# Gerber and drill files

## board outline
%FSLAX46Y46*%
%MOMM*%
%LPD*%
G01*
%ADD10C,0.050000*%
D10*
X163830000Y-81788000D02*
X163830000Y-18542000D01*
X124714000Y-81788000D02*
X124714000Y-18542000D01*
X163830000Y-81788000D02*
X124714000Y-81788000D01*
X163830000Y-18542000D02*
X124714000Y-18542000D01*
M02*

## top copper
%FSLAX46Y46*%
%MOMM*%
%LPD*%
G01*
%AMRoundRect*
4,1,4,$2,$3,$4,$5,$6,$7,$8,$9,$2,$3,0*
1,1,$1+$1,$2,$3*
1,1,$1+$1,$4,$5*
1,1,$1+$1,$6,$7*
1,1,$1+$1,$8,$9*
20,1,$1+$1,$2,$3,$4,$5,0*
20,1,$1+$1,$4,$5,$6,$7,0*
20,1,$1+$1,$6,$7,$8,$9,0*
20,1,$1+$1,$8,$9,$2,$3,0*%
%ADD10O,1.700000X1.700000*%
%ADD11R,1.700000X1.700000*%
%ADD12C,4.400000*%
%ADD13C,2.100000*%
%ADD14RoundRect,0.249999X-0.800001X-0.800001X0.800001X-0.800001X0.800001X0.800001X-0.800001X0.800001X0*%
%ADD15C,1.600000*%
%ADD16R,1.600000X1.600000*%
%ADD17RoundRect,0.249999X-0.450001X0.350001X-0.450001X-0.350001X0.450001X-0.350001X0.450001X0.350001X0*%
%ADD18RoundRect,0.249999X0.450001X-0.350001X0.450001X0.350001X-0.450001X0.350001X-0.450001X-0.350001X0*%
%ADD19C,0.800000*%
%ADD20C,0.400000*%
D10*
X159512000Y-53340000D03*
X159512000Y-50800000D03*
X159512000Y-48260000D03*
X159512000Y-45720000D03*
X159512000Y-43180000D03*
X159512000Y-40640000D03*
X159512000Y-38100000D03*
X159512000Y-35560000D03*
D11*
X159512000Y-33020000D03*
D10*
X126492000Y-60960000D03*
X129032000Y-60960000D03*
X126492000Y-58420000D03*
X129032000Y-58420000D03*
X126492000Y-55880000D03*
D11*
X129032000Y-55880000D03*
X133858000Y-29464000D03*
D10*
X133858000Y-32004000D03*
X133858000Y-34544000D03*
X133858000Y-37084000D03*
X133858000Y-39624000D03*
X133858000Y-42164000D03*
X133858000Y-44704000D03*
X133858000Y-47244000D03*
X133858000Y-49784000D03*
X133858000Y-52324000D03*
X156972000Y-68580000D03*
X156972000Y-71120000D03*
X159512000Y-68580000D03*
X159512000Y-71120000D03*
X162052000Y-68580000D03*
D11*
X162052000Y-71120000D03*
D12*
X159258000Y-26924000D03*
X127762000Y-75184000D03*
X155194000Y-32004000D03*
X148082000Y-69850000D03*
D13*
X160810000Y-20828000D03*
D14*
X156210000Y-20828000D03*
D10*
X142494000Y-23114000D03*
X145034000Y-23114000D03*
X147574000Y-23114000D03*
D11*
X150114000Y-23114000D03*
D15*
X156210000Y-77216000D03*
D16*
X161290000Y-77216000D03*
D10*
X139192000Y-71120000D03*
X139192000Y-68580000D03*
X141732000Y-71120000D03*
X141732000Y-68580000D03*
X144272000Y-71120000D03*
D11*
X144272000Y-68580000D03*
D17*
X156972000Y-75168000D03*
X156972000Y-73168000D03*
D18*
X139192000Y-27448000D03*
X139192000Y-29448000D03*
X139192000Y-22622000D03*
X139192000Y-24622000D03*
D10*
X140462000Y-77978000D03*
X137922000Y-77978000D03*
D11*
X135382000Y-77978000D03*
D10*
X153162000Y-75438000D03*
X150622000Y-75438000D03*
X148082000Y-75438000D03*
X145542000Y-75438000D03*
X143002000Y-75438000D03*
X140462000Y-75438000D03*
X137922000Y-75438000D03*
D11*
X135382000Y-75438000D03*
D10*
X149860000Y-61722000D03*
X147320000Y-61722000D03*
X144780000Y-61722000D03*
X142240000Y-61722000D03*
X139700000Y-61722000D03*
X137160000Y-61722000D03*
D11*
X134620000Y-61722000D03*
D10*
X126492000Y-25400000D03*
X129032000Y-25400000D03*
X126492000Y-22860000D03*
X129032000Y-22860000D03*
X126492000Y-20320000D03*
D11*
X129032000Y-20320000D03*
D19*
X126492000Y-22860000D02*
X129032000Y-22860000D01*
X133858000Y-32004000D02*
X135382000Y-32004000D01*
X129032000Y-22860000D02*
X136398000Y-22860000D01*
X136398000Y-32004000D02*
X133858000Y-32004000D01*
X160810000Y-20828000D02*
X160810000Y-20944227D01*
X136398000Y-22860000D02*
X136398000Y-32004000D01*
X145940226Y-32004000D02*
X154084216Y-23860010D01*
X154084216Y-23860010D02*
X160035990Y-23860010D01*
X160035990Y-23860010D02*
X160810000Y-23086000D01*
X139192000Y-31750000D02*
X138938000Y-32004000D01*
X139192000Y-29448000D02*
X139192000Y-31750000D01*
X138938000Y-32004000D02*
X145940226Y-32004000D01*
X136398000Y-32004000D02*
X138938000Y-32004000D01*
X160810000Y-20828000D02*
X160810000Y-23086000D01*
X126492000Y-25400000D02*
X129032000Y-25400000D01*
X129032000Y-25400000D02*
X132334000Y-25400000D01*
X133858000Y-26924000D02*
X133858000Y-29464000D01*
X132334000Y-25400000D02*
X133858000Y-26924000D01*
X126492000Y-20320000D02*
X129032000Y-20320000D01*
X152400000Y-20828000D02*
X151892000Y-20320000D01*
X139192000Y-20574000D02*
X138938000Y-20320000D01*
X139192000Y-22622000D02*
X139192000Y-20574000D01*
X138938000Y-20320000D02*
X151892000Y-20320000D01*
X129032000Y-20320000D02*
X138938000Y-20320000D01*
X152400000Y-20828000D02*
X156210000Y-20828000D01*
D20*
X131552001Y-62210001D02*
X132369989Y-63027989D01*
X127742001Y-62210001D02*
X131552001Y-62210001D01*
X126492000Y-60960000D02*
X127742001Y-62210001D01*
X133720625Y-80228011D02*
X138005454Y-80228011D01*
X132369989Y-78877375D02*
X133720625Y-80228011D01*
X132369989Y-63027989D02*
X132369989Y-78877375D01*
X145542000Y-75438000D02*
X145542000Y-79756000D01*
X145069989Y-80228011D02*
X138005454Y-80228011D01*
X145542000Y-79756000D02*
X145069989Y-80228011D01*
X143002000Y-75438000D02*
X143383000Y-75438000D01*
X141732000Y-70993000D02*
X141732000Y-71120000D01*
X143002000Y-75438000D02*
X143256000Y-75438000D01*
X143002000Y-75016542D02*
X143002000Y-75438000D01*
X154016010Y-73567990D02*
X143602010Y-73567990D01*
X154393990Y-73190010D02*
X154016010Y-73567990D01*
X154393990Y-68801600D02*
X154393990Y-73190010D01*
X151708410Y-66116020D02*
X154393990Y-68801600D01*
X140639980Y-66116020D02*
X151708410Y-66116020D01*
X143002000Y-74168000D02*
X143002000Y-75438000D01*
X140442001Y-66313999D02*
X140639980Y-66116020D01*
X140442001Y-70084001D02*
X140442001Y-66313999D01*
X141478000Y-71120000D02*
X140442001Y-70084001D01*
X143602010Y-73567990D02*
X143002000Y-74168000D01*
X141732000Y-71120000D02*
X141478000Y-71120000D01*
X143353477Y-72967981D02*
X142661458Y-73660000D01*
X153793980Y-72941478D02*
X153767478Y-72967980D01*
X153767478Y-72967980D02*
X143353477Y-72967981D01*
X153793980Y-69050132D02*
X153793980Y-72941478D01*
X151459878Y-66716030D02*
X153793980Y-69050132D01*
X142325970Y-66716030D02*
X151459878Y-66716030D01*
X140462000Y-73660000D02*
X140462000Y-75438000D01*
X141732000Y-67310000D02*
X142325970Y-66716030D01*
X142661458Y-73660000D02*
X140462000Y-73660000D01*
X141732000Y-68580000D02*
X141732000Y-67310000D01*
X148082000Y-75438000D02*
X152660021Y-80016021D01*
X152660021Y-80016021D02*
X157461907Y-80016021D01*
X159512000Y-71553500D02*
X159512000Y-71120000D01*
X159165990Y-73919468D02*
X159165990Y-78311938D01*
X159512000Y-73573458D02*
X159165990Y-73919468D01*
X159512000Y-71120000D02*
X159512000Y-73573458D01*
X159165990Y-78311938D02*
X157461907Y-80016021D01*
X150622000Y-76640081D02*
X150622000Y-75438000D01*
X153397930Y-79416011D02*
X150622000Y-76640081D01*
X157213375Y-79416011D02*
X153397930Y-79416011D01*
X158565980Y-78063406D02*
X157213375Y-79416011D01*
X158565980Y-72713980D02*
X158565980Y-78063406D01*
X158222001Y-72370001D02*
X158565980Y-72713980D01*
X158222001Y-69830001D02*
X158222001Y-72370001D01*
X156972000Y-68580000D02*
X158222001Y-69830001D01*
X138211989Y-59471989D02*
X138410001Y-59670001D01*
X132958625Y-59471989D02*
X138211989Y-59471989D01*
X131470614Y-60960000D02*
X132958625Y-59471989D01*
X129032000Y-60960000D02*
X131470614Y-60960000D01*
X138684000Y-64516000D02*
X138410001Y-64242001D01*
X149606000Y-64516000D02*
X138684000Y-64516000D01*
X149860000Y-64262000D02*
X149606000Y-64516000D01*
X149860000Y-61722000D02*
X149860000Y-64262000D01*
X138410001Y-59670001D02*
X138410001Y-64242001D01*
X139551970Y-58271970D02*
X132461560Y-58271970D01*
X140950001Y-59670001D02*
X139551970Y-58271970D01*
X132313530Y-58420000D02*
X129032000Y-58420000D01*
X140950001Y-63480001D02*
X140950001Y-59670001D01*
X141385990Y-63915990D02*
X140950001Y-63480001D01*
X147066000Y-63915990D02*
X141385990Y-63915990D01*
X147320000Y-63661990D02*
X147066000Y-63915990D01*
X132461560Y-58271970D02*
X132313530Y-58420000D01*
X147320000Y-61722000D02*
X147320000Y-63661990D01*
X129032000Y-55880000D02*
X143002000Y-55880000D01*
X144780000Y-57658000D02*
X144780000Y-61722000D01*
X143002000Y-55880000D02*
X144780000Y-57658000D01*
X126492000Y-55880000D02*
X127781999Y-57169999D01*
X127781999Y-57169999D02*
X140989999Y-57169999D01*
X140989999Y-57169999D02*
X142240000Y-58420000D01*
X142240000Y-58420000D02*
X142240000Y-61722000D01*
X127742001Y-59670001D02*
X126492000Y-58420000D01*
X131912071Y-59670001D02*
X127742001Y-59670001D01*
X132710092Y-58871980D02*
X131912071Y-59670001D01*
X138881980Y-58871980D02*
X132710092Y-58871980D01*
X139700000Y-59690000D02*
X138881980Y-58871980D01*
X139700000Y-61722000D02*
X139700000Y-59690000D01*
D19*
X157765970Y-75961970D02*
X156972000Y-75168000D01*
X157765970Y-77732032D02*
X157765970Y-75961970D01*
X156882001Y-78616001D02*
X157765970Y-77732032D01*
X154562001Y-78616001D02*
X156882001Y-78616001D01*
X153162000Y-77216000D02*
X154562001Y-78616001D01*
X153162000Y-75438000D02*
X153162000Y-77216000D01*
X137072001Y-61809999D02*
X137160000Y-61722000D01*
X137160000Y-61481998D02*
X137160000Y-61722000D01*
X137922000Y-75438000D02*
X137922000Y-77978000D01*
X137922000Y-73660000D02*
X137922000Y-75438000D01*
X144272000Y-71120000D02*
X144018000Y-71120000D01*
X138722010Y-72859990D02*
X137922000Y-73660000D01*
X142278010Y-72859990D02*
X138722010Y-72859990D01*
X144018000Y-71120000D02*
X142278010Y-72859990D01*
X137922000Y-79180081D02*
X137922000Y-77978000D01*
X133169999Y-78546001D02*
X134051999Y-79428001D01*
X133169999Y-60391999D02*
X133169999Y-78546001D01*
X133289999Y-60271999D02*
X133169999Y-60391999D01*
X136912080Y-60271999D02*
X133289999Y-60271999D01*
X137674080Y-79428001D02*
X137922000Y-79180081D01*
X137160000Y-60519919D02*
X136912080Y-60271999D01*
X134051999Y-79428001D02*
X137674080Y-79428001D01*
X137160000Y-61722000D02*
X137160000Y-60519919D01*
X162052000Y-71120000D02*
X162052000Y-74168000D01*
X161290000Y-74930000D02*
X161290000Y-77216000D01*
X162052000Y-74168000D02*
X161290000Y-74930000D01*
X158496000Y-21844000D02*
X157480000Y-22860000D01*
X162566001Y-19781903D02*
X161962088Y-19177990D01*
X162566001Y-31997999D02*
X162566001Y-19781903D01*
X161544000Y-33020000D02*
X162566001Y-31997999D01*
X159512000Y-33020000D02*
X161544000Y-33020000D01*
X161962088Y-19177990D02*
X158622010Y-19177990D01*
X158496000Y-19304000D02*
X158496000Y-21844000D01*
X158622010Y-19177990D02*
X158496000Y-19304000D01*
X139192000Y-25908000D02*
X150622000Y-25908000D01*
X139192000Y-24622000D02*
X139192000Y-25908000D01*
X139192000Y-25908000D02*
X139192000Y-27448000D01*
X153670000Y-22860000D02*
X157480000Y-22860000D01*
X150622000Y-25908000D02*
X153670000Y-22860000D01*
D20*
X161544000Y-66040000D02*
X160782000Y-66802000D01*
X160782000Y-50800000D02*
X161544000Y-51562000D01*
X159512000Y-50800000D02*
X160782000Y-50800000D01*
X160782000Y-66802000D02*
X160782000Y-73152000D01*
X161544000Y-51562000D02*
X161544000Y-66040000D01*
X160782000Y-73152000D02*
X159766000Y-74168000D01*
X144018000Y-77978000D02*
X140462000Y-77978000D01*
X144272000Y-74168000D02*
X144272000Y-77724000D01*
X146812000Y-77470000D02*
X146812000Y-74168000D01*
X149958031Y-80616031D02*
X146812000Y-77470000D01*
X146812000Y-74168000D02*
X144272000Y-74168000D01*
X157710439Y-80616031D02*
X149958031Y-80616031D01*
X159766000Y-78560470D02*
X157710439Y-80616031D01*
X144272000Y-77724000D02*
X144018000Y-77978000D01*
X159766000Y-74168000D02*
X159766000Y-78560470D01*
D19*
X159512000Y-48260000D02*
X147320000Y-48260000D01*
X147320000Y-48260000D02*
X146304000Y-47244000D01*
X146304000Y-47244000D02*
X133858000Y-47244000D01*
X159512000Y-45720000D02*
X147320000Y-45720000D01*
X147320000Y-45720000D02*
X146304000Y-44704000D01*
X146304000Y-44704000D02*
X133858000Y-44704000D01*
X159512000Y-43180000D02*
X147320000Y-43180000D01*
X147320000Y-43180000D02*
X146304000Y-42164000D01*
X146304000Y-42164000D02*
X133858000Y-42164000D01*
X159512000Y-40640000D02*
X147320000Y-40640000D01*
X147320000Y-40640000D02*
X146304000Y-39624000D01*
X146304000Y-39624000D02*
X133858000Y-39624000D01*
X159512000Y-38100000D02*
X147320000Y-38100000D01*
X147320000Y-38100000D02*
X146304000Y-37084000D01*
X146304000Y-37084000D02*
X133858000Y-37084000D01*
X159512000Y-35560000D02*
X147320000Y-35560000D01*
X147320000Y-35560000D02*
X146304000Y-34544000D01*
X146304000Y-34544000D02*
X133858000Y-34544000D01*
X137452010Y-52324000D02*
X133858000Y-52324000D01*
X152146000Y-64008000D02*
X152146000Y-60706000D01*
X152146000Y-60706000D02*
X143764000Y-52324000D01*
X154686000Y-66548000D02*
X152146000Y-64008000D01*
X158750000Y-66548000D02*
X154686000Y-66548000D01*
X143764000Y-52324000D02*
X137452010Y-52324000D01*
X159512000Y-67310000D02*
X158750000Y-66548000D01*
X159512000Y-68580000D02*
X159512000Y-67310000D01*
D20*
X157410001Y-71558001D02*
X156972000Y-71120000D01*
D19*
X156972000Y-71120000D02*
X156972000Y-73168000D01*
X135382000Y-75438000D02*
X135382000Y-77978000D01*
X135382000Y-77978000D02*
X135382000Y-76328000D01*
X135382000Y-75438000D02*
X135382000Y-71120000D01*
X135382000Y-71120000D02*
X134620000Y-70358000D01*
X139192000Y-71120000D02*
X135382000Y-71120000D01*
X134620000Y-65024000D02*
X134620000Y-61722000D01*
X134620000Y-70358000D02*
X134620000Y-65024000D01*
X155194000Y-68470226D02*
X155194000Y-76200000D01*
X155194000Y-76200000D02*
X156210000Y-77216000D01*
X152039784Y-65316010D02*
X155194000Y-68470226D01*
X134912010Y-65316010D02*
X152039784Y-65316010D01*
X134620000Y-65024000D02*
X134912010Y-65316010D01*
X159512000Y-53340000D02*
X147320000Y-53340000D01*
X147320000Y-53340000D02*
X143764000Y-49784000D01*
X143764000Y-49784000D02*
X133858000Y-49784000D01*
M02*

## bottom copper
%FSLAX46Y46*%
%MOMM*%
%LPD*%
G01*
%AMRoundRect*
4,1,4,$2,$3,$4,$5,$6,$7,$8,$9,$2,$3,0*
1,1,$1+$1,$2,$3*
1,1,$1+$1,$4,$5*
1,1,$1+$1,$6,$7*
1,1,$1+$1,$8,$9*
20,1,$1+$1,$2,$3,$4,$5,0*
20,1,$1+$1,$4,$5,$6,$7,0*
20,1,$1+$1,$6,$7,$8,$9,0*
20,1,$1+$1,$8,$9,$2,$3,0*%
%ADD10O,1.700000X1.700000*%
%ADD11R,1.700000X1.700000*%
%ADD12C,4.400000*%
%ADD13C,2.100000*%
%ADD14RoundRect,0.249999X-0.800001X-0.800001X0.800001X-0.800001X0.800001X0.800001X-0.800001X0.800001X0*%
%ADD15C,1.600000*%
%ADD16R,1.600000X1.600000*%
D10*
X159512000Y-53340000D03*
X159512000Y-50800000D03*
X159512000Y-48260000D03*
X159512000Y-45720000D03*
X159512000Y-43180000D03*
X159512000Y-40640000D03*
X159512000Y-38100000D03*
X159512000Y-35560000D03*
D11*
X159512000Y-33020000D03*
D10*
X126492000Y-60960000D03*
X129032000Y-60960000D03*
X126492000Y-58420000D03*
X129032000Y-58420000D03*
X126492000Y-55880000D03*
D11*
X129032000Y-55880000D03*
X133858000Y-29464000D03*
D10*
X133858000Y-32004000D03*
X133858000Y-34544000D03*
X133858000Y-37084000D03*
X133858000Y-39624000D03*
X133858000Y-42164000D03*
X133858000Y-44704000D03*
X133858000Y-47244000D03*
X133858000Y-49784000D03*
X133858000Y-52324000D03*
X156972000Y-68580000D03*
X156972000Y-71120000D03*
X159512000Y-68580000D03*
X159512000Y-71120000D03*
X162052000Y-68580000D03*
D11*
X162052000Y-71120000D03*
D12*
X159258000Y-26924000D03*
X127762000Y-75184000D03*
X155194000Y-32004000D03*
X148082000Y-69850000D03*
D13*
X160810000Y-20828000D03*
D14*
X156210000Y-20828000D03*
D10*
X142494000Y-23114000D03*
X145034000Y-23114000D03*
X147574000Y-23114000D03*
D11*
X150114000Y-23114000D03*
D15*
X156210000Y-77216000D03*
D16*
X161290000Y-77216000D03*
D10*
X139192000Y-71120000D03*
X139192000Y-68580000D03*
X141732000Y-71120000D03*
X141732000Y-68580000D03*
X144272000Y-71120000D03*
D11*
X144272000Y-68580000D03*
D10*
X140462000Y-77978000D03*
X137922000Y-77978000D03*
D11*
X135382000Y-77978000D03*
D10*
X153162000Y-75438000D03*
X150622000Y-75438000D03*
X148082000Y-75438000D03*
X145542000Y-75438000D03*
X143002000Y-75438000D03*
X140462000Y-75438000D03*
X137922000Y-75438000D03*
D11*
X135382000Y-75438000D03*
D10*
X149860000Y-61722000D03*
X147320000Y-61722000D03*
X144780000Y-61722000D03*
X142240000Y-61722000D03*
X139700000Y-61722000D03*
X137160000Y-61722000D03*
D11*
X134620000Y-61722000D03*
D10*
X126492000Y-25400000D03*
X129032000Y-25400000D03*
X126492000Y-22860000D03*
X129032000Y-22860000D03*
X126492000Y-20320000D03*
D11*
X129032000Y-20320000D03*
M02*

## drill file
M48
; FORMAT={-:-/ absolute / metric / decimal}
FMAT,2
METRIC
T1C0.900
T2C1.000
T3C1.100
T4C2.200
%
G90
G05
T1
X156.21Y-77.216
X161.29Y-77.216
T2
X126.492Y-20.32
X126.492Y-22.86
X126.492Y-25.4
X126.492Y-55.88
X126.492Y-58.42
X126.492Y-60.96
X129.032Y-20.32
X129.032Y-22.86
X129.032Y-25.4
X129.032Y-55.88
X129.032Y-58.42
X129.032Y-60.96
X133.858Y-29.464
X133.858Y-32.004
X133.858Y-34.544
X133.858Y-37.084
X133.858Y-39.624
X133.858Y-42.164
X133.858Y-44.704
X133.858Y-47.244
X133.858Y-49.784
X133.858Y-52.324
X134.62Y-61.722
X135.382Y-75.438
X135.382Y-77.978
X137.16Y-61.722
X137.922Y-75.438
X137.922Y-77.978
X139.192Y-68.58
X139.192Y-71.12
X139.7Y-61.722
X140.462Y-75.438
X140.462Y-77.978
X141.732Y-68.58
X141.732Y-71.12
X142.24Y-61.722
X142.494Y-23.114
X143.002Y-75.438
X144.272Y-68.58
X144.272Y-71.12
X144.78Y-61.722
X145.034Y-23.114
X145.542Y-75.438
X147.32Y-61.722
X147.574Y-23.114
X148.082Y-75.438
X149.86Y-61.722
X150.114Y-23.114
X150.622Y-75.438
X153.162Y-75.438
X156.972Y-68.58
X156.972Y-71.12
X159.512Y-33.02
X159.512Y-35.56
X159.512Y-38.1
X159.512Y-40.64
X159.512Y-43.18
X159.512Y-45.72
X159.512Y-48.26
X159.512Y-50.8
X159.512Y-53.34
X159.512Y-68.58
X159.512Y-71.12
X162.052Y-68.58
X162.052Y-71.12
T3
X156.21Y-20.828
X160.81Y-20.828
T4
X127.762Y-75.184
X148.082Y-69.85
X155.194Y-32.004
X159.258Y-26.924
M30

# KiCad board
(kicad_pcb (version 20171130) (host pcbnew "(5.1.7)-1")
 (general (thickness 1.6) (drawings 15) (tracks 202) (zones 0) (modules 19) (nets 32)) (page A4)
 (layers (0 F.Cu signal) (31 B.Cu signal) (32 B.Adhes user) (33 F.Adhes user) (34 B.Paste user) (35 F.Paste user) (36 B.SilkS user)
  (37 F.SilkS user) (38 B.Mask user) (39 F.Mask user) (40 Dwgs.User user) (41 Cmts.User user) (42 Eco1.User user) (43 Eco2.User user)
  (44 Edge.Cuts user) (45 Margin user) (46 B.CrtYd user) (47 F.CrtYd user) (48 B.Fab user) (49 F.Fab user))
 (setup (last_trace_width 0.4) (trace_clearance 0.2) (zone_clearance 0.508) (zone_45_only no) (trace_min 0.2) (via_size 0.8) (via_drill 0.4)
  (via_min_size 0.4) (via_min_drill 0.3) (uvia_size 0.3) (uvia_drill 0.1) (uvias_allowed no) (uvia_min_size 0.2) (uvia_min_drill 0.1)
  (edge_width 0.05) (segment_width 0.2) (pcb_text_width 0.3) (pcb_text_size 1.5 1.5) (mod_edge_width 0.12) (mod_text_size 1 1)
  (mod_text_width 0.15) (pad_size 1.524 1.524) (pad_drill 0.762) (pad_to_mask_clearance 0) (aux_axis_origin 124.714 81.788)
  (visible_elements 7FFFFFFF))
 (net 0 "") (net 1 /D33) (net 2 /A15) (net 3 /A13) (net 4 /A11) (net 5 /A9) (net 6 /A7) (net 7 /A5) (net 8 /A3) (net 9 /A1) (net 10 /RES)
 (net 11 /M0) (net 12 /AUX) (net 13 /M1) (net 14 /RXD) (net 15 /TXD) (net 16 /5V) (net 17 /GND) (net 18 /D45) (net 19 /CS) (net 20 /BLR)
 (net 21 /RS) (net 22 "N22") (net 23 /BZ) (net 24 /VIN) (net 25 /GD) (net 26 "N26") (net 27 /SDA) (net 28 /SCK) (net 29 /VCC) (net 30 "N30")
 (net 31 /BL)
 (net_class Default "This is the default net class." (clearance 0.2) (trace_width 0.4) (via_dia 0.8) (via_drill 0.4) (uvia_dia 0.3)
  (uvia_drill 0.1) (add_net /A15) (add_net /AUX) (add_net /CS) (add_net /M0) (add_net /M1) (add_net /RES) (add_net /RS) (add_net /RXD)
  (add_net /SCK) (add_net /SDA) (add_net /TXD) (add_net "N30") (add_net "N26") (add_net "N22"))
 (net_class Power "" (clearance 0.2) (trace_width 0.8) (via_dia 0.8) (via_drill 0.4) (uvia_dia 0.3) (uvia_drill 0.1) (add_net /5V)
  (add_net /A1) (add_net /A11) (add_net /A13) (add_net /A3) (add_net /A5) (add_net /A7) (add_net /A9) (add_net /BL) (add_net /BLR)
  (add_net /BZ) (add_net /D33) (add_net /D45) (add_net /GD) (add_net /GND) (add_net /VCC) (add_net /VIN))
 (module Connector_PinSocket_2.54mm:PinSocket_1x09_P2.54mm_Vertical (layer F.Cu) (at 159.512 33.02)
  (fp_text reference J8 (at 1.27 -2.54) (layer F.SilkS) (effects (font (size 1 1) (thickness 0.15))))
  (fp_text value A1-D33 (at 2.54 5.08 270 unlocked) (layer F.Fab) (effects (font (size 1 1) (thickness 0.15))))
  (pad 9 thru_hole oval (at 0 20.32) (size 1.7 1.7) (drill 1) (layers *.Cu *.Mask) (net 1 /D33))
  (pad 8 thru_hole oval (at 0 17.78) (size 1.7 1.7) (drill 1) (layers *.Cu *.Mask) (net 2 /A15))
  (pad 7 thru_hole oval (at 0 15.24) (size 1.7 1.7) (drill 1) (layers *.Cu *.Mask) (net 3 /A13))
  (pad 6 thru_hole oval (at 0 12.7) (size 1.7 1.7) (drill 1) (layers *.Cu *.Mask) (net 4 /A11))
  (pad 5 thru_hole oval (at 0 10.16) (size 1.7 1.7) (drill 1) (layers *.Cu *.Mask) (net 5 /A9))
  (pad 4 thru_hole oval (at 0 7.62) (size 1.7 1.7) (drill 1) (layers *.Cu *.Mask) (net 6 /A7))
  (pad 3 thru_hole oval (at 0 5.08) (size 1.7 1.7) (drill 1) (layers *.Cu *.Mask) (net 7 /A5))
  (pad 2 thru_hole oval (at 0 2.54) (size 1.7 1.7) (drill 1) (layers *.Cu *.Mask) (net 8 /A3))
  (pad 1 thru_hole rect (at 0 0) (size 1.7 1.7) (drill 1) (layers *.Cu *.Mask) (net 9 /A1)))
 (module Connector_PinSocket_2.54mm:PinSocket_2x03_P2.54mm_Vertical (layer F.Cu) (at 129.032 55.88)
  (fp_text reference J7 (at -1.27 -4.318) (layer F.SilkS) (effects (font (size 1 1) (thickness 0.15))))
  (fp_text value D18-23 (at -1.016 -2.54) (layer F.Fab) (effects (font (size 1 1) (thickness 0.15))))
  (pad 6 thru_hole oval (at -2.54 5.08) (size 1.7 1.7) (drill 1) (layers *.Cu *.Mask) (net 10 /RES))
  (pad 5 thru_hole oval (at 0 5.08) (size 1.7 1.7) (drill 1) (layers *.Cu *.Mask) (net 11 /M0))
  (pad 4 thru_hole oval (at -2.54 2.54) (size 1.7 1.7) (drill 1) (layers *.Cu *.Mask) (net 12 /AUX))
  (pad 3 thru_hole oval (at 0 2.54) (size 1.7 1.7) (drill 1) (layers *.Cu *.Mask) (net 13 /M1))
  (pad 2 thru_hole oval (at -2.54 0) (size 1.7 1.7) (drill 1) (layers *.Cu *.Mask) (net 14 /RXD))
  (pad 1 thru_hole rect (at 0 0) (size 1.7 1.7) (drill 1) (layers *.Cu *.Mask) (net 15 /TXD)))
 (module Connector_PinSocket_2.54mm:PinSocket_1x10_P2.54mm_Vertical (layer F.Cu) (at 133.858 29.464)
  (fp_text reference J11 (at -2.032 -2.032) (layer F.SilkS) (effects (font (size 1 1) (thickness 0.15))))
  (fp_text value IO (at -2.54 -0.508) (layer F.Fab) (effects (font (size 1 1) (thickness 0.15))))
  (pad 1 thru_hole rect (at 0 0) (size 1.7 1.7) (drill 1) (layers *.Cu *.Mask) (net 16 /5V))
  (pad 2 thru_hole oval (at 0 2.54) (size 1.7 1.7) (drill 1) (layers *.Cu *.Mask) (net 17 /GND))
  (pad 3 thru_hole oval (at 0 5.08) (size 1.7 1.7) (drill 1) (layers *.Cu *.Mask) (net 8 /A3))
  (pad 4 thru_hole oval (at 0 7.62) (size 1.7 1.7) (drill 1) (layers *.Cu *.Mask) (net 7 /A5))
  (pad 5 thru_hole oval (at 0 10.16) (size 1.7 1.7) (drill 1) (layers *.Cu *.Mask) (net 6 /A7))
  (pad 6 thru_hole oval (at 0 12.7) (size 1.7 1.7) (drill 1) (layers *.Cu *.Mask) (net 5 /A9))
  (pad 7 thru_hole oval (at 0 15.24) (size 1.7 1.7) (drill 1) (layers *.Cu *.Mask) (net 4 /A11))
  (pad 8 thru_hole oval (at 0 17.78) (size 1.7 1.7) (drill 1) (layers *.Cu *.Mask) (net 3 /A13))
  (pad 9 thru_hole oval (at 0 20.32) (size 1.7 1.7) (drill 1) (layers *.Cu *.Mask) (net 1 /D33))
  (pad 10 thru_hole oval (at 0 22.86) (size 1.7 1.7) (drill 1) (layers *.Cu *.Mask) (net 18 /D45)))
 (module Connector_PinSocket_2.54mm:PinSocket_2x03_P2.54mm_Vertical (layer F.Cu) (at 162.052 71.12 270)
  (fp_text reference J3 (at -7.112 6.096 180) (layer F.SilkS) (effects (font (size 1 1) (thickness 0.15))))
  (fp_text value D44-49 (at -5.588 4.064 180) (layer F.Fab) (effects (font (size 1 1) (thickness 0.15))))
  (pad 6 thru_hole oval (at -2.54 5.08 270) (size 1.7 1.7) (drill 1) (layers *.Cu *.Mask) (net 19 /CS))
  (pad 5 thru_hole oval (at 0 5.08 270) (size 1.7 1.7) (drill 1) (layers *.Cu *.Mask) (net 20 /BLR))
  (pad 4 thru_hole oval (at -2.54 2.54 270) (size 1.7 1.7) (drill 1) (layers *.Cu *.Mask) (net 18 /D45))
  (pad 3 thru_hole oval (at 0 2.54 270) (size 1.7 1.7) (drill 1) (layers *.Cu *.Mask) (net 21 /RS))
  (pad 2 thru_hole oval (at -2.54 0 270) (size 1.7 1.7) (drill 1) (layers *.Cu *.Mask) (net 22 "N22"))
  (pad 1 thru_hole rect (at 0 0 270) (size 1.7 1.7) (drill 1) (layers *.Cu *.Mask) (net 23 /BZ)))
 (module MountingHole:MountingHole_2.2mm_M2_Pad (layer F.Cu) (at 159.258 26.924)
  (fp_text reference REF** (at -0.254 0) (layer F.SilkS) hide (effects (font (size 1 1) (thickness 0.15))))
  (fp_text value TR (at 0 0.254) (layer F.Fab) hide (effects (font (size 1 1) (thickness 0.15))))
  (pad 1 thru_hole circle (at 0 0) (size 4.4 4.4) (drill 2.2) (layers *.Cu *.Mask)))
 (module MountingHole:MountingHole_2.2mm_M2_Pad (layer F.Cu) (at 127.762 75.184)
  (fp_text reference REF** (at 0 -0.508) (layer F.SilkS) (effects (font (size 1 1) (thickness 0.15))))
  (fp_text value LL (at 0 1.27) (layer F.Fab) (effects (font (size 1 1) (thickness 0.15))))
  (pad 1 thru_hole circle (at 0 0) (size 4.4 4.4) (drill 2.2) (layers *.Cu *.Mask)))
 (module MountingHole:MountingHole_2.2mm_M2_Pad (layer F.Cu) (at 155.194 32.004)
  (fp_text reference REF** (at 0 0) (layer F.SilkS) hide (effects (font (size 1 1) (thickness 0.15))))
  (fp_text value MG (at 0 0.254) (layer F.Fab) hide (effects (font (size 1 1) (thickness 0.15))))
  (pad 1 thru_hole circle (at 0 0) (size 4.4 4.4) (drill 2.2) (layers *.Cu *.Mask)))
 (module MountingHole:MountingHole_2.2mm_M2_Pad (layer F.Cu) (at 148.082 69.85)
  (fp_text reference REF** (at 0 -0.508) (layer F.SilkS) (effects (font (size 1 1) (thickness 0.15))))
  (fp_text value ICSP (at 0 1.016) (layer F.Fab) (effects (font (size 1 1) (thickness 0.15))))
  (pad 1 thru_hole circle (at 0 0) (size 4.4 4.4) (drill 2.2) (layers *.Cu *.Mask)))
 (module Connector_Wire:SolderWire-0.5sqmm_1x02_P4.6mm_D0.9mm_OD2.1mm (layer F.Cu) (at 156.21 20.828)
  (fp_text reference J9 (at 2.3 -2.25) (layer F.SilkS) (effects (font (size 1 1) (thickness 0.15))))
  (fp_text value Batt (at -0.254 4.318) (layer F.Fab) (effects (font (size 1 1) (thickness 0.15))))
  (pad 2 thru_hole circle (at 4.6 0) (size 2.1 2.1) (drill 1.1) (layers *.Cu *.Mask) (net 17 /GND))
  (pad 1 thru_hole roundrect (at 0 0) (size 2.1 2.1) (drill 1.1) (layers *.Cu *.Mask) (roundrect_rratio 0.1190471428571429) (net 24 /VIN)))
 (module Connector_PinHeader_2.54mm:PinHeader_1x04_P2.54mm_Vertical (layer F.Cu) (at 150.114 23.114 270)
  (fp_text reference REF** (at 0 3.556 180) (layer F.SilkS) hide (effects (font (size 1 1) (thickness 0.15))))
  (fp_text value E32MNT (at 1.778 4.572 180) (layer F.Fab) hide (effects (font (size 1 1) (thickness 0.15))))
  (pad 4 thru_hole oval (at 0 7.62 270) (size 1.7 1.7) (drill 1) (layers *.Cu *.Mask))
  (pad 3 thru_hole oval (at 0 5.08 270) (size 1.7 1.7) (drill 1) (layers *.Cu *.Mask))
  (pad 2 thru_hole oval (at 0 2.54 270) (size 1.7 1.7) (drill 1) (layers *.Cu *.Mask))
  (pad 1 thru_hole rect (at 0 0 270) (size 1.7 1.7) (drill 1) (layers *.Cu *.Mask)))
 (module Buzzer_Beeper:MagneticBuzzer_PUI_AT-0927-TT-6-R (layer F.Cu) (at 160.782 77.216 180)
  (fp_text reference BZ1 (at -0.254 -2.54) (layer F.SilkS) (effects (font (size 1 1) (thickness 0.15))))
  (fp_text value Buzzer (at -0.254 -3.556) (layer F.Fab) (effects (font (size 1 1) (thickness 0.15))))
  (pad 2 thru_hole circle (at 4.572 0 180) (size 1.6 1.6) (drill 0.9) (layers *.Cu *.Mask) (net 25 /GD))
  (pad 1 thru_hole rect (at -0.508 0 180) (size 1.6 1.6) (drill 0.9) (layers *.Cu *.Mask) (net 23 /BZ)))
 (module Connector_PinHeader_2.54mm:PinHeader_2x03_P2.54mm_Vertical (layer F.Cu) (at 144.272 68.58 270)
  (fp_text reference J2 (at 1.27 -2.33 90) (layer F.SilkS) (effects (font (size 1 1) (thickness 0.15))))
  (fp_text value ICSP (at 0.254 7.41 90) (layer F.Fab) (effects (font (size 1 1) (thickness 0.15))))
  (pad 6 thru_hole oval (at 2.54 5.08 270) (size 1.7 1.7) (drill 1) (layers *.Cu *.Mask) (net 25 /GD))
  (pad 5 thru_hole oval (at 0 5.08 270) (size 1.7 1.7) (drill 1) (layers *.Cu *.Mask) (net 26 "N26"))
  (pad 4 thru_hole oval (at 2.54 2.54 270) (size 1.7 1.7) (drill 1) (layers *.Cu *.Mask) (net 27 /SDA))
  (pad 3 thru_hole oval (at 0 2.54 270) (size 1.7 1.7) (drill 1) (layers *.Cu *.Mask) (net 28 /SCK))
  (pad 2 thru_hole oval (at 2.54 0 270) (size 1.7 1.7) (drill 1) (layers *.Cu *.Mask) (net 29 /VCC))
  (pad 1 thru_hole rect (at 0 0 270) (size 1.7 1.7) (drill 1) (layers *.Cu *.Mask) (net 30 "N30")))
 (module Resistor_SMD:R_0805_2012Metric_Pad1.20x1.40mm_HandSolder (layer F.Cu) (at 156.972 74.168 270)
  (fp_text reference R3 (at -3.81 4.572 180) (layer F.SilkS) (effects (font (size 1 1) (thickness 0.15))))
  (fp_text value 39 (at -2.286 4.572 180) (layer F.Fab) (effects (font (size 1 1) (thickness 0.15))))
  (pad 2 smd roundrect (at 1 0 270) (size 1.2 1.4) (layers F.Cu F.Paste F.Mask) (roundrect_rratio 0.2083325) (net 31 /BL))
  (pad 1 smd roundrect (at -1 0 270) (size 1.2 1.4) (layers F.Cu F.Paste F.Mask) (roundrect_rratio 0.2083325) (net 20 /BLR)))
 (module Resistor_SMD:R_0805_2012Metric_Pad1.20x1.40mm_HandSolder (layer F.Cu) (at 139.192 28.448 90)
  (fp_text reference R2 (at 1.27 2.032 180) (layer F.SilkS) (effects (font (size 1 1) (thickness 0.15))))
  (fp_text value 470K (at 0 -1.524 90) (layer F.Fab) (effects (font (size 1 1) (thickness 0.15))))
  (pad 2 smd roundrect (at 1 0 90) (size 1.2 1.4) (layers F.Cu F.Paste F.Mask) (roundrect_rratio 0.2083325) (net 9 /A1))
  (pad 1 smd roundrect (at -1 0 90) (size 1.2 1.4) (layers F.Cu F.Paste F.Mask) (roundrect_rratio 0.2083325) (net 17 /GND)))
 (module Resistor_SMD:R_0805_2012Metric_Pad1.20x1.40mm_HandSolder (layer F.Cu) (at 139.192 23.622 90)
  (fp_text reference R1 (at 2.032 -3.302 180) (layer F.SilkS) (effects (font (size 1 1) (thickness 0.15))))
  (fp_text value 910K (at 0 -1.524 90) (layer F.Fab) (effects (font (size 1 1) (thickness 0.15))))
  (pad 2 smd roundrect (at 1 0 90) (size 1.2 1.4) (layers F.Cu F.Paste F.Mask) (roundrect_rratio 0.2083325) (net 24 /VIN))
  (pad 1 smd roundrect (at -1 0 90) (size 1.2 1.4) (layers F.Cu F.Paste F.Mask) (roundrect_rratio 0.2083325) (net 9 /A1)))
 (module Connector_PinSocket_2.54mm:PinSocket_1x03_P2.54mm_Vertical (layer F.Cu) (at 135.382 77.978 90)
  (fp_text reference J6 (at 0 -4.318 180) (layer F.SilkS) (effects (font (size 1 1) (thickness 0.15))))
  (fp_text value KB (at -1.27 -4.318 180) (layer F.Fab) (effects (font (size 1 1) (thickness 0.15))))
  (pad 3 thru_hole oval (at 0 5.08 90) (size 1.7 1.7) (drill 1) (layers *.Cu *.Mask) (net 2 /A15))
  (pad 2 thru_hole oval (at 0 2.54 90) (size 1.7 1.7) (drill 1) (layers *.Cu *.Mask) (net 29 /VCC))
  (pad 1 thru_hole rect (at 0 0 90) (size 1.7 1.7) (drill 1) (layers *.Cu *.Mask) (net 25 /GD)))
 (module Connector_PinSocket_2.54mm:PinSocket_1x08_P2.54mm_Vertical (layer F.Cu) (at 135.382 75.438 90)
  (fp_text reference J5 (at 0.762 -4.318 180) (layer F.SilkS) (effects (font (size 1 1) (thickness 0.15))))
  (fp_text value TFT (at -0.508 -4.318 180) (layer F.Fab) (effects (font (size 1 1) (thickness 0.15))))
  (pad 8 thru_hole oval (at 0 17.78 90) (size 1.7 1.7) (drill 1) (layers *.Cu *.Mask) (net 31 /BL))
  (pad 7 thru_hole oval (at 0 15.24 90) (size 1.7 1.7) (drill 1) (layers *.Cu *.Mask) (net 19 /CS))
  (pad 6 thru_hole oval (at 0 12.7 90) (size 1.7 1.7) (drill 1) (layers *.Cu *.Mask) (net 21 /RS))
  (pad 5 thru_hole oval (at 0 10.16 90) (size 1.7 1.7) (drill 1) (layers *.Cu *.Mask) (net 10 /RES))
  (pad 4 thru_hole oval (at 0 7.62 90) (size 1.7 1.7) (drill 1) (layers *.Cu *.Mask) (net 27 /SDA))
  (pad 3 thru_hole oval (at 0 5.08 90) (size 1.7 1.7) (drill 1) (layers *.Cu *.Mask) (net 28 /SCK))
  (pad 2 thru_hole oval (at 0 2.54 90) (size 1.7 1.7) (drill 1) (layers *.Cu *.Mask) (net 29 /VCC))
  (pad 1 thru_hole rect (at 0 0 90) (size 1.7 1.7) (drill 1) (layers *.Cu *.Mask) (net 25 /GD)))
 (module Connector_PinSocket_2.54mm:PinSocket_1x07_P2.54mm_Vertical (layer F.Cu) (at 134.62 61.722 90)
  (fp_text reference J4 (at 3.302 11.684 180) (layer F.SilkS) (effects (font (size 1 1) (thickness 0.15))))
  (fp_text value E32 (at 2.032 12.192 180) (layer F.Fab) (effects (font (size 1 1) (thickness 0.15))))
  (pad 7 thru_hole oval (at 0 15.24 90) (size 1.7 1.7) (drill 1) (layers *.Cu *.Mask) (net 11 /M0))
  (pad 6 thru_hole oval (at 0 12.7 90) (size 1.7 1.7) (drill 1) (layers *.Cu *.Mask) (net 13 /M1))
  (pad 5 thru_hole oval (at 0 10.16 90) (size 1.7 1.7) (drill 1) (layers *.Cu *.Mask) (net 15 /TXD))
  (pad 4 thru_hole oval (at 0 7.62 90) (size 1.7 1.7) (drill 1) (layers *.Cu *.Mask) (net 14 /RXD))
  (pad 3 thru_hole oval (at 0 5.08 90) (size 1.7 1.7) (drill 1) (layers *.Cu *.Mask) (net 12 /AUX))
  (pad 2 thru_hole oval (at 0 2.54 90) (size 1.7 1.7) (drill 1) (layers *.Cu *.Mask) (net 29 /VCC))
  (pad 1 thru_hole rect (at 0 0 90) (size 1.7 1.7) (drill 1) (layers *.Cu *.Mask) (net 25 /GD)))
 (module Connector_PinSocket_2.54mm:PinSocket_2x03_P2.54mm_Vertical (layer F.Cu) (at 129.032 20.32)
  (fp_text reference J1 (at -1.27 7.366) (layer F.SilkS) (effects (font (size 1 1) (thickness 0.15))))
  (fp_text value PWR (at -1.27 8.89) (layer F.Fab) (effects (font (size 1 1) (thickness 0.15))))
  (pad 6 thru_hole oval (at -2.54 5.08) (size 1.7 1.7) (drill 1) (layers *.Cu *.Mask) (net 16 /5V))
  (pad 5 thru_hole oval (at 0 5.08) (size 1.7 1.7) (drill 1) (layers *.Cu *.Mask) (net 16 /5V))
  (pad 4 thru_hole oval (at -2.54 2.54) (size 1.7 1.7) (drill 1) (layers *.Cu *.Mask) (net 17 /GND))
  (pad 3 thru_hole oval (at 0 2.54) (size 1.7 1.7) (drill 1) (layers *.Cu *.Mask) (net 17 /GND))
  (pad 2 thru_hole oval (at -2.54 0) (size 1.7 1.7) (drill 1) (layers *.Cu *.Mask) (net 24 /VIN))
  (pad 1 thru_hole rect (at 0 0) (size 1.7 1.7) (drill 1) (layers *.Cu *.Mask) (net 24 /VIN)))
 (gr_line (start 163.83 81.788) (end 163.83 18.542) (layer Edge.Cuts) (width 0.05))
 (gr_line (start 124.714 81.788) (end 124.714 18.542) (layer Edge.Cuts) (width 0.05))
 (gr_line (start 163.83 81.788) (end 124.714 81.788) (layer Edge.Cuts) (width 0.05))
 (gr_line (start 163.83 18.542) (end 124.714 18.542) (layer Edge.Cuts) (width 0.05))
 (segment (start 126.492 22.86) (end 129.032 22.86) (width 0.8) (layer F.Cu) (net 17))
 (segment (start 133.858 32.004) (end 135.382 32.004) (width 0.8) (layer F.Cu) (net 17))
 (segment (start 129.032 22.86) (end 136.398 22.86) (width 0.8) (layer F.Cu) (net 17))
 (segment (start 136.398 32.004) (end 133.858 32.004) (width 0.8) (layer F.Cu) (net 17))
 (segment (start 160.81 20.828) (end 160.81 20.944227) (width 0.8) (layer F.Cu) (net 17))
 (segment (start 136.398 22.86) (end 136.398 32.004) (width 0.8) (layer F.Cu) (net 17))
 (segment (start 145.940226 32.004) (end 154.084216 23.86001) (width 0.8) (layer F.Cu) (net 17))
 (segment (start 154.084216 23.86001) (end 160.03599 23.86001) (width 0.8) (layer F.Cu) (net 17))
 (segment (start 160.03599 23.86001) (end 160.81 23.086) (width 0.8) (layer F.Cu) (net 17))
 (segment (start 139.192 31.75) (end 138.938 32.004) (width 0.8) (layer F.Cu) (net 17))
 (segment (start 139.192 29.448) (end 139.192 31.75) (width 0.8) (layer F.Cu) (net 17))
 (segment (start 138.938 32.004) (end 145.940226 32.004) (width 0.8) (layer F.Cu) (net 17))
 (segment (start 136.398 32.004) (end 138.938 32.004) (width 0.8) (layer F.Cu) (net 17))
 (segment (start 160.81 20.828) (end 160.81 23.086) (width 0.8) (layer F.Cu) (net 17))
 (segment (start 126.492 25.4) (end 129.032 25.4) (width 0.8) (layer F.Cu) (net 16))
 (segment (start 129.032 25.4) (end 132.334 25.4) (width 0.8) (layer F.Cu) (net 16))
 (segment (start 133.858 26.924) (end 133.858 29.464) (width 0.8) (layer F.Cu) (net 16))
 (segment (start 132.334 25.4) (end 133.858 26.924) (width 0.8) (layer F.Cu) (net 16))
 (segment (start 126.492 20.32) (end 129.032 20.32) (width 0.8) (layer F.Cu) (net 24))
 (segment (start 152.4 20.828) (end 151.892 20.32) (width 0.8) (layer F.Cu) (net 24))
 (segment (start 139.192 20.574) (end 138.938 20.32) (width 0.8) (layer F.Cu) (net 24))
 (segment (start 139.192 22.622) (end 139.192 20.574) (width 0.8) (layer F.Cu) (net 24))
 (segment (start 138.938 20.32) (end 151.892 20.32) (width 0.8) (layer F.Cu) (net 24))
 (segment (start 129.032 20.32) (end 138.938 20.32) (width 0.8) (layer F.Cu) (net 24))
 (segment (start 152.4 20.828) (end 156.21 20.828) (width 0.8) (layer F.Cu) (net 24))
 (segment (start 131.552001 62.210001) (end 132.369989 63.027989) (width 0.4) (layer F.Cu) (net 10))
 (segment (start 127.742001 62.210001) (end 131.552001 62.210001) (width 0.4) (layer F.Cu) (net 10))
 (segment (start 126.492 60.96) (end 127.742001 62.210001) (width 0.4) (layer F.Cu) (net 10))
 (segment (start 133.720625 80.228011) (end 138.005454 80.228011) (width 0.4) (layer F.Cu) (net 10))
 (segment (start 132.369989 78.877375) (end 133.720625 80.228011) (width 0.4) (layer F.Cu) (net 10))
 (segment (start 132.369989 63.027989) (end 132.369989 78.877375) (width 0.4) (layer F.Cu) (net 10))
 (segment (start 145.542 75.438) (end 145.542 79.756) (width 0.4) (layer F.Cu) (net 10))
 (segment (start 145.069989 80.228011) (end 138.005454 80.228011) (width 0.4) (layer F.Cu) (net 10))
 (segment (start 145.542 79.756) (end 145.069989 80.228011) (width 0.4) (layer F.Cu) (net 10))
 (segment (start 143.002 75.438) (end 143.383 75.438) (width 0.4) (layer F.Cu) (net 27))
 (segment (start 141.732 70.993) (end 141.732 71.12) (width 0.4) (layer F.Cu) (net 27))
 (segment (start 143.002 75.438) (end 143.256 75.438) (width 0.4) (layer F.Cu) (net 27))
 (segment (start 143.002 75.016542) (end 143.002 75.438) (width 0.4) (layer F.Cu) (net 27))
 (segment (start 154.01601 73.56799) (end 143.60201 73.56799) (width 0.4) (layer F.Cu) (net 27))
 (segment (start 154.39399 73.19001) (end 154.01601 73.56799) (width 0.4) (layer F.Cu) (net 27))
 (segment (start 154.39399 68.8016) (end 154.39399 73.19001) (width 0.4) (layer F.Cu) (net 27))
 (segment (start 151.70841 66.11602) (end 154.39399 68.8016) (width 0.4) (layer F.Cu) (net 27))
 (segment (start 140.63998 66.11602) (end 151.70841 66.11602) (width 0.4) (layer F.Cu) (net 27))
 (segment (start 143.002 74.168) (end 143.002 75.438) (width 0.4) (layer F.Cu) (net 27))
 (segment (start 140.442001 66.313999) (end 140.63998 66.11602) (width 0.4) (layer F.Cu) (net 27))
 (segment (start 140.442001 70.084001) (end 140.442001 66.313999) (width 0.4) (layer F.Cu) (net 27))
 (segment (start 141.478 71.12) (end 140.442001 70.084001) (width 0.4) (layer F.Cu) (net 27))
 (segment (start 143.60201 73.56799) (end 143.002 74.168) (width 0.4) (layer F.Cu) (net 27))
 (segment (start 141.732 71.12) (end 141.478 71.12) (width 0.4) (layer F.Cu) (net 27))
 (segment (start 143.353477 72.967981) (end 142.661458 73.66) (width 0.4) (layer F.Cu) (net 28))
 (segment (start 153.79398 72.941478) (end 153.767478 72.96798) (width 0.4) (layer F.Cu) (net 28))
 (segment (start 153.767478 72.96798) (end 143.353477 72.967981) (width 0.4) (layer F.Cu) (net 28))
 (segment (start 153.79398 69.050132) (end 153.79398 72.941478) (width 0.4) (layer F.Cu) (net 28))
 (segment (start 151.459878 66.71603) (end 153.79398 69.050132) (width 0.4) (layer F.Cu) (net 28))
 (segment (start 142.32597 66.71603) (end 151.459878 66.71603) (width 0.4) (layer F.Cu) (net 28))
 (segment (start 140.462 73.66) (end 140.462 75.438) (width 0.4) (layer F.Cu) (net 28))
 (segment (start 141.732 67.31) (end 142.32597 66.71603) (width 0.4) (layer F.Cu) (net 28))
 (segment (start 142.661458 73.66) (end 140.462 73.66) (width 0.4) (layer F.Cu) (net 28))
 (segment (start 141.732 68.58) (end 141.732 67.31) (width 0.4) (layer F.Cu) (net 28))
 (segment (start 148.082 75.438) (end 152.660021 80.016021) (width 0.4) (layer F.Cu) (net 21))
 (segment (start 152.660021 80.016021) (end 157.461907 80.016021) (width 0.4) (layer F.Cu) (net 21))
 (segment (start 159.512 71.5535) (end 159.512 71.12) (width 0.4) (layer F.Cu) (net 21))
 (segment (start 159.16599 73.919468) (end 159.16599 78.311938) (width 0.4) (layer F.Cu) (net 21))
 (segment (start 159.512 73.573458) (end 159.16599 73.919468) (width 0.4) (layer F.Cu) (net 21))
 (segment (start 159.512 71.12) (end 159.512 73.573458) (width 0.4) (layer F.Cu) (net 21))
 (segment (start 159.16599 78.311938) (end 157.461907 80.016021) (width 0.4) (layer F.Cu) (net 21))
 (segment (start 150.622 76.640081) (end 150.622 75.438) (width 0.4) (layer F.Cu) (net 19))
 (segment (start 153.39793 79.416011) (end 150.622 76.640081) (width 0.4) (layer F.Cu) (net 19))
 (segment (start 157.213375 79.416011) (end 153.39793 79.416011) (width 0.4) (layer F.Cu) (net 19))
 (segment (start 158.56598 78.063406) (end 157.213375 79.416011) (width 0.4) (layer F.Cu) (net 19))
 (segment (start 158.56598 72.71398) (end 158.56598 78.063406) (width 0.4) (layer F.Cu) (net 19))
 (segment (start 158.222001 72.370001) (end 158.56598 72.71398) (width 0.4) (layer F.Cu) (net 19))
 (segment (start 158.222001 69.830001) (end 158.222001 72.370001) (width 0.4) (layer F.Cu) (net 19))
 (segment (start 156.972 68.58) (end 158.222001 69.830001) (width 0.4) (layer F.Cu) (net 19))
 (segment (start 138.211989 59.471989) (end 138.410001 59.670001) (width 0.4) (layer F.Cu) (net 11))
 (segment (start 132.958625 59.471989) (end 138.211989 59.471989) (width 0.4) (layer F.Cu) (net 11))
 (segment (start 131.470614 60.96) (end 132.958625 59.471989) (width 0.4) (layer F.Cu) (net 11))
 (segment (start 129.032 60.96) (end 131.470614 60.96) (width 0.4) (layer F.Cu) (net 11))
 (segment (start 138.684 64.516) (end 138.410001 64.242001) (width 0.4) (layer F.Cu) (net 11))
 (segment (start 149.606 64.516) (end 138.684 64.516) (width 0.4) (layer F.Cu) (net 11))
 (segment (start 149.86 64.262) (end 149.606 64.516) (width 0.4) (layer F.Cu) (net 11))
 (segment (start 149.86 61.722) (end 149.86 64.262) (width 0.4) (layer F.Cu) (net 11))
 (segment (start 138.410001 59.670001) (end 138.410001 64.242001) (width 0.4) (layer F.Cu) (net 11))
 (segment (start 139.55197 58.27197) (end 132.46156 58.27197) (width 0.4) (layer F.Cu) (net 13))
 (segment (start 140.950001 59.670001) (end 139.55197 58.27197) (width 0.4) (layer F.Cu) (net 13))
 (segment (start 132.31353 58.42) (end 129.032 58.42) (width 0.4) (layer F.Cu) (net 13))
 (segment (start 140.950001 63.480001) (end 140.950001 59.670001) (width 0.4) (layer F.Cu) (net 13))
 (segment (start 141.38599 63.91599) (end 140.950001 63.480001) (width 0.4) (layer F.Cu) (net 13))
 (segment (start 147.066 63.91599) (end 141.38599 63.91599) (width 0.4) (layer F.Cu) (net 13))
 (segment (start 147.32 63.66199) (end 147.066 63.91599) (width 0.4) (layer F.Cu) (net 13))
 (segment (start 132.46156 58.27197) (end 132.31353 58.42) (width 0.4) (layer F.Cu) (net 13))
 (segment (start 147.32 61.722) (end 147.32 63.66199) (width 0.4) (layer F.Cu) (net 13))
 (segment (start 129.032 55.88) (end 143.002 55.88) (width 0.4) (layer F.Cu) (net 15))
 (segment (start 144.78 57.658) (end 144.78 61.722) (width 0.4) (layer F.Cu) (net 15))
 (segment (start 143.002 55.88) (end 144.78 57.658) (width 0.4) (layer F.Cu) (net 15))
 (segment (start 126.492 55.88) (end 127.781999 57.169999) (width 0.4) (layer F.Cu) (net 14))
 (segment (start 127.781999 57.169999) (end 140.989999 57.169999) (width 0.4) (layer F.Cu) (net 14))
 (segment (start 140.989999 57.169999) (end 142.24 58.42) (width 0.4) (layer F.Cu) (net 14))
 (segment (start 142.24 58.42) (end 142.24 61.722) (width 0.4) (layer F.Cu) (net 14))
 (segment (start 127.742001 59.670001) (end 126.492 58.42) (width 0.4) (layer F.Cu) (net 12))
 (segment (start 131.912071 59.670001) (end 127.742001 59.670001) (width 0.4) (layer F.Cu) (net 12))
 (segment (start 132.710092 58.87198) (end 131.912071 59.670001) (width 0.4) (layer F.Cu) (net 12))
 (segment (start 138.88198 58.87198) (end 132.710092 58.87198) (width 0.4) (layer F.Cu) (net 12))
 (segment (start 139.7 59.69) (end 138.88198 58.87198) (width 0.4) (layer F.Cu) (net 12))
 (segment (start 139.7 61.722) (end 139.7 59.69) (width 0.4) (layer F.Cu) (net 12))
 (segment (start 157.76597 75.96197) (end 156.972 75.168) (width 0.8) (layer F.Cu) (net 31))
 (segment (start 157.76597 77.732032) (end 157.76597 75.96197) (width 0.8) (layer F.Cu) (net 31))
 (segment (start 156.882001 78.616001) (end 157.76597 77.732032) (width 0.8) (layer F.Cu) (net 31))
 (segment (start 154.562001 78.616001) (end 156.882001 78.616001) (width 0.8) (layer F.Cu) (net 31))
 (segment (start 153.162 77.216) (end 154.562001 78.616001) (width 0.8) (layer F.Cu) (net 31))
 (segment (start 153.162 75.438) (end 153.162 77.216) (width 0.8) (layer F.Cu) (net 31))
 (segment (start 137.072001 61.809999) (end 137.16 61.722) (width 0.8) (layer F.Cu) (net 29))
 (segment (start 137.16 61.481998) (end 137.16 61.722) (width 0.8) (layer F.Cu) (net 29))
 (segment (start 137.922 75.438) (end 137.922 77.978) (width 0.8) (layer F.Cu) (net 29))
 (segment (start 137.922 73.66) (end 137.922 75.438) (width 0.8) (layer F.Cu) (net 29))
 (segment (start 144.272 71.12) (end 144.018 71.12) (width 0.8) (layer F.Cu) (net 29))
 (segment (start 138.72201 72.85999) (end 137.922 73.66) (width 0.8) (layer F.Cu) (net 29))
 (segment (start 142.27801 72.85999) (end 138.72201 72.85999) (width 0.8) (layer F.Cu) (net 29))
 (segment (start 144.018 71.12) (end 142.27801 72.85999) (width 0.8) (layer F.Cu) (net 29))
 (segment (start 137.922 79.180081) (end 137.922 77.978) (width 0.8) (layer F.Cu) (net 29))
 (segment (start 133.169999 78.546001) (end 134.051999 79.428001) (width 0.8) (layer F.Cu) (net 29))
 (segment (start 133.169999 60.391999) (end 133.169999 78.546001) (width 0.8) (layer F.Cu) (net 29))
 (segment (start 133.289999 60.271999) (end 133.169999 60.391999) (width 0.8) (layer F.Cu) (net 29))
 (segment (start 136.91208 60.271999) (end 133.289999 60.271999) (width 0.8) (layer F.Cu) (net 29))
 (segment (start 137.67408 79.428001) (end 137.922 79.180081) (width 0.8) (layer F.Cu) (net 29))
 (segment (start 137.16 60.519919) (end 136.91208 60.271999) (width 0.8) (layer F.Cu) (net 29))
 (segment (start 134.051999 79.428001) (end 137.67408 79.428001) (width 0.8) (layer F.Cu) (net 29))
 (segment (start 137.16 61.722) (end 137.16 60.519919) (width 0.8) (layer F.Cu) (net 29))
 (segment (start 162.052 71.12) (end 162.052 74.168) (width 0.8) (layer F.Cu) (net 23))
 (segment (start 161.29 74.93) (end 161.29 77.216) (width 0.8) (layer F.Cu) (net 23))
 (segment (start 162.052 74.168) (end 161.29 74.93) (width 0.8) (layer F.Cu) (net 23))
 (segment (start 158.496 21.844) (end 157.48 22.86) (width 0.8) (layer F.Cu) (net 9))
 (segment (start 162.566001 19.781903) (end 161.962088 19.17799) (width 0.8) (layer F.Cu) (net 9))
 (segment (start 162.566001 31.997999) (end 162.566001 19.781903) (width 0.8) (layer F.Cu) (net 9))
 (segment (start 161.544 33.02) (end 162.566001 31.997999) (width 0.8) (layer F.Cu) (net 9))
 (segment (start 159.512 33.02) (end 161.544 33.02) (width 0.8) (layer F.Cu) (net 9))
 (segment (start 161.962088 19.17799) (end 158.62201 19.17799) (width 0.8) (layer F.Cu) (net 9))
 (segment (start 158.496 19.304) (end 158.496 21.844) (width 0.8) (layer F.Cu) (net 9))
 (segment (start 158.62201 19.17799) (end 158.496 19.304) (width 0.8) (layer F.Cu) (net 9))
 (segment (start 139.192 25.908) (end 150.622 25.908) (width 0.8) (layer F.Cu) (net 9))
 (segment (start 139.192 24.622) (end 139.192 25.908) (width 0.8) (layer F.Cu) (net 9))
 (segment (start 139.192 25.908) (end 139.192 27.448) (width 0.8) (layer F.Cu) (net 9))
 (segment (start 153.67 22.86) (end 157.48 22.86) (width 0.8) (layer F.Cu) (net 9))
 (segment (start 150.622 25.908) (end 153.67 22.86) (width 0.8) (layer F.Cu) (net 9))
 (segment (start 161.544 66.04) (end 160.782 66.802) (width 0.4) (layer F.Cu) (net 2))
 (segment (start 160.782 50.8) (end 161.544 51.562) (width 0.4) (layer F.Cu) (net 2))
 (segment (start 159.512 50.8) (end 160.782 50.8) (width 0.4) (layer F.Cu) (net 2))
 (segment (start 160.782 66.802) (end 160.782 73.152) (width 0.4) (layer F.Cu) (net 2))
 (segment (start 161.544 51.562) (end 161.544 66.04) (width 0.4) (layer F.Cu) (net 2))
 (segment (start 160.782 73.152) (end 159.766 74.168) (width 0.4) (layer F.Cu) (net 2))
 (segment (start 144.018 77.978) (end 140.462 77.978) (width 0.4) (layer F.Cu) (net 2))
 (segment (start 144.272 74.168) (end 144.272 77.724) (width 0.4) (layer F.Cu) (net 2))
 (segment (start 146.812 77.47) (end 146.812 74.168) (width 0.4) (layer F.Cu) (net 2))
 (segment (start 149.958031 80.616031) (end 146.812 77.47) (width 0.4) (layer F.Cu) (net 2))
 (segment (start 146.812 74.168) (end 144.272 74.168) (width 0.4) (layer F.Cu) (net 2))
 (segment (start 157.710439 80.616031) (end 149.958031 80.616031) (width 0.4) (layer F.Cu) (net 2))
 (segment (start 159.766 78.56047) (end 157.710439 80.616031) (width 0.4) (layer F.Cu) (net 2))
 (segment (start 144.272 77.724) (end 144.018 77.978) (width 0.4) (layer F.Cu) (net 2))
 (segment (start 159.766 74.168) (end 159.766 78.56047) (width 0.4) (layer F.Cu) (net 2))
 (segment (start 159.512 48.26) (end 147.32 48.26) (width 0.8) (layer F.Cu) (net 3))
 (segment (start 147.32 48.26) (end 146.304 47.244) (width 0.8) (layer F.Cu) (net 3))
 (segment (start 146.304 47.244) (end 133.858 47.244) (width 0.8) (layer F.Cu) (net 3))
 (segment (start 159.512 45.72) (end 147.32 45.72) (width 0.8) (layer F.Cu) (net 4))
 (segment (start 147.32 45.72) (end 146.304 44.704) (width 0.8) (layer F.Cu) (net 4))
 (segment (start 146.304 44.704) (end 133.858 44.704) (width 0.8) (layer F.Cu) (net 4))
 (segment (start 159.512 43.18) (end 147.32 43.18) (width 0.8) (layer F.Cu) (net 5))
 (segment (start 147.32 43.18) (end 146.304 42.164) (width 0.8) (layer F.Cu) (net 5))
 (segment (start 146.304 42.164) (end 133.858 42.164) (width 0.8) (layer F.Cu) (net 5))
 (segment (start 159.512 40.64) (end 147.32 40.64) (width 0.8) (layer F.Cu) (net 6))
 (segment (start 147.32 40.64) (end 146.304 39.624) (width 0.8) (layer F.Cu) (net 6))
 (segment (start 146.304 39.624) (end 133.858 39.624) (width 0.8) (layer F.Cu) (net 6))
 (segment (start 159.512 38.1) (end 147.32 38.1) (width 0.8) (layer F.Cu) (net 7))
 (segment (start 147.32 38.1) (end 146.304 37.084) (width 0.8) (layer F.Cu) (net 7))
 (segment (start 146.304 37.084) (end 133.858 37.084) (width 0.8) (layer F.Cu) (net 7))
 (segment (start 159.512 35.56) (end 147.32 35.56) (width 0.8) (layer F.Cu) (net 8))
 (segment (start 147.32 35.56) (end 146.304 34.544) (width 0.8) (layer F.Cu) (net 8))
 (segment (start 146.304 34.544) (end 133.858 34.544) (width 0.8) (layer F.Cu) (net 8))
 (segment (start 137.45201 52.324) (end 133.858 52.324) (width 0.8) (layer F.Cu) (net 18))
 (segment (start 152.146 64.008) (end 152.146 60.706) (width 0.8) (layer F.Cu) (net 18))
 (segment (start 152.146 60.706) (end 143.764 52.324) (width 0.8) (layer F.Cu) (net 18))
 (segment (start 154.686 66.548) (end 152.146 64.008) (width 0.8) (layer F.Cu) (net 18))
 (segment (start 158.75 66.548) (end 154.686 66.548) (width 0.8) (layer F.Cu) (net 18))
 (segment (start 143.764 52.324) (end 137.45201 52.324) (width 0.8) (layer F.Cu) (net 18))
 (segment (start 159.512 67.31) (end 158.75 66.548) (width 0.8) (layer F.Cu) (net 18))
 (segment (start 159.512 68.58) (end 159.512 67.31) (width 0.8) (layer F.Cu) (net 18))
 (segment (start 157.410001 71.558001) (end 156.972 71.12) (width 0.4) (layer F.Cu) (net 20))
 (segment (start 156.972 71.12) (end 156.972 73.168) (width 0.8) (layer F.Cu) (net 20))
 (segment (start 135.382 75.438) (end 135.382 77.978) (width 0.8) (layer F.Cu) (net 25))
 (segment (start 135.382 77.978) (end 135.382 76.328) (width 0.8) (layer F.Cu) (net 25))
 (segment (start 135.382 75.438) (end 135.382 71.12) (width 0.8) (layer F.Cu) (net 25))
 (segment (start 135.382 71.12) (end 134.62 70.358) (width 0.8) (layer F.Cu) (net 25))
 (segment (start 139.192 71.12) (end 135.382 71.12) (width 0.8) (layer F.Cu) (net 25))
 (segment (start 134.62 65.024) (end 134.62 61.722) (width 0.8) (layer F.Cu) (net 25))
 (segment (start 134.62 70.358) (end 134.62 65.024) (width 0.8) (layer F.Cu) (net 25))
 (segment (start 155.194 68.470226) (end 155.194 76.2) (width 0.8) (layer F.Cu) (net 25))
 (segment (start 155.194 76.2) (end 156.21 77.216) (width 0.8) (layer F.Cu) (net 25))
 (segment (start 152.039784 65.31601) (end 155.194 68.470226) (width 0.8) (layer F.Cu) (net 25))
 (segment (start 134.91201 65.31601) (end 152.039784 65.31601) (width 0.8) (layer F.Cu) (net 25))
 (segment (start 134.62 65.024) (end 134.91201 65.31601) (width 0.8) (layer F.Cu) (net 25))
 (segment (start 159.512 53.34) (end 147.32 53.34) (width 0.8) (layer F.Cu) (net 1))
 (segment (start 147.32 53.34) (end 143.764 49.784) (width 0.8) (layer F.Cu) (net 1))
 (segment (start 143.764 49.784) (end 133.858 49.784) (width 0.8) (layer F.Cu) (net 1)))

